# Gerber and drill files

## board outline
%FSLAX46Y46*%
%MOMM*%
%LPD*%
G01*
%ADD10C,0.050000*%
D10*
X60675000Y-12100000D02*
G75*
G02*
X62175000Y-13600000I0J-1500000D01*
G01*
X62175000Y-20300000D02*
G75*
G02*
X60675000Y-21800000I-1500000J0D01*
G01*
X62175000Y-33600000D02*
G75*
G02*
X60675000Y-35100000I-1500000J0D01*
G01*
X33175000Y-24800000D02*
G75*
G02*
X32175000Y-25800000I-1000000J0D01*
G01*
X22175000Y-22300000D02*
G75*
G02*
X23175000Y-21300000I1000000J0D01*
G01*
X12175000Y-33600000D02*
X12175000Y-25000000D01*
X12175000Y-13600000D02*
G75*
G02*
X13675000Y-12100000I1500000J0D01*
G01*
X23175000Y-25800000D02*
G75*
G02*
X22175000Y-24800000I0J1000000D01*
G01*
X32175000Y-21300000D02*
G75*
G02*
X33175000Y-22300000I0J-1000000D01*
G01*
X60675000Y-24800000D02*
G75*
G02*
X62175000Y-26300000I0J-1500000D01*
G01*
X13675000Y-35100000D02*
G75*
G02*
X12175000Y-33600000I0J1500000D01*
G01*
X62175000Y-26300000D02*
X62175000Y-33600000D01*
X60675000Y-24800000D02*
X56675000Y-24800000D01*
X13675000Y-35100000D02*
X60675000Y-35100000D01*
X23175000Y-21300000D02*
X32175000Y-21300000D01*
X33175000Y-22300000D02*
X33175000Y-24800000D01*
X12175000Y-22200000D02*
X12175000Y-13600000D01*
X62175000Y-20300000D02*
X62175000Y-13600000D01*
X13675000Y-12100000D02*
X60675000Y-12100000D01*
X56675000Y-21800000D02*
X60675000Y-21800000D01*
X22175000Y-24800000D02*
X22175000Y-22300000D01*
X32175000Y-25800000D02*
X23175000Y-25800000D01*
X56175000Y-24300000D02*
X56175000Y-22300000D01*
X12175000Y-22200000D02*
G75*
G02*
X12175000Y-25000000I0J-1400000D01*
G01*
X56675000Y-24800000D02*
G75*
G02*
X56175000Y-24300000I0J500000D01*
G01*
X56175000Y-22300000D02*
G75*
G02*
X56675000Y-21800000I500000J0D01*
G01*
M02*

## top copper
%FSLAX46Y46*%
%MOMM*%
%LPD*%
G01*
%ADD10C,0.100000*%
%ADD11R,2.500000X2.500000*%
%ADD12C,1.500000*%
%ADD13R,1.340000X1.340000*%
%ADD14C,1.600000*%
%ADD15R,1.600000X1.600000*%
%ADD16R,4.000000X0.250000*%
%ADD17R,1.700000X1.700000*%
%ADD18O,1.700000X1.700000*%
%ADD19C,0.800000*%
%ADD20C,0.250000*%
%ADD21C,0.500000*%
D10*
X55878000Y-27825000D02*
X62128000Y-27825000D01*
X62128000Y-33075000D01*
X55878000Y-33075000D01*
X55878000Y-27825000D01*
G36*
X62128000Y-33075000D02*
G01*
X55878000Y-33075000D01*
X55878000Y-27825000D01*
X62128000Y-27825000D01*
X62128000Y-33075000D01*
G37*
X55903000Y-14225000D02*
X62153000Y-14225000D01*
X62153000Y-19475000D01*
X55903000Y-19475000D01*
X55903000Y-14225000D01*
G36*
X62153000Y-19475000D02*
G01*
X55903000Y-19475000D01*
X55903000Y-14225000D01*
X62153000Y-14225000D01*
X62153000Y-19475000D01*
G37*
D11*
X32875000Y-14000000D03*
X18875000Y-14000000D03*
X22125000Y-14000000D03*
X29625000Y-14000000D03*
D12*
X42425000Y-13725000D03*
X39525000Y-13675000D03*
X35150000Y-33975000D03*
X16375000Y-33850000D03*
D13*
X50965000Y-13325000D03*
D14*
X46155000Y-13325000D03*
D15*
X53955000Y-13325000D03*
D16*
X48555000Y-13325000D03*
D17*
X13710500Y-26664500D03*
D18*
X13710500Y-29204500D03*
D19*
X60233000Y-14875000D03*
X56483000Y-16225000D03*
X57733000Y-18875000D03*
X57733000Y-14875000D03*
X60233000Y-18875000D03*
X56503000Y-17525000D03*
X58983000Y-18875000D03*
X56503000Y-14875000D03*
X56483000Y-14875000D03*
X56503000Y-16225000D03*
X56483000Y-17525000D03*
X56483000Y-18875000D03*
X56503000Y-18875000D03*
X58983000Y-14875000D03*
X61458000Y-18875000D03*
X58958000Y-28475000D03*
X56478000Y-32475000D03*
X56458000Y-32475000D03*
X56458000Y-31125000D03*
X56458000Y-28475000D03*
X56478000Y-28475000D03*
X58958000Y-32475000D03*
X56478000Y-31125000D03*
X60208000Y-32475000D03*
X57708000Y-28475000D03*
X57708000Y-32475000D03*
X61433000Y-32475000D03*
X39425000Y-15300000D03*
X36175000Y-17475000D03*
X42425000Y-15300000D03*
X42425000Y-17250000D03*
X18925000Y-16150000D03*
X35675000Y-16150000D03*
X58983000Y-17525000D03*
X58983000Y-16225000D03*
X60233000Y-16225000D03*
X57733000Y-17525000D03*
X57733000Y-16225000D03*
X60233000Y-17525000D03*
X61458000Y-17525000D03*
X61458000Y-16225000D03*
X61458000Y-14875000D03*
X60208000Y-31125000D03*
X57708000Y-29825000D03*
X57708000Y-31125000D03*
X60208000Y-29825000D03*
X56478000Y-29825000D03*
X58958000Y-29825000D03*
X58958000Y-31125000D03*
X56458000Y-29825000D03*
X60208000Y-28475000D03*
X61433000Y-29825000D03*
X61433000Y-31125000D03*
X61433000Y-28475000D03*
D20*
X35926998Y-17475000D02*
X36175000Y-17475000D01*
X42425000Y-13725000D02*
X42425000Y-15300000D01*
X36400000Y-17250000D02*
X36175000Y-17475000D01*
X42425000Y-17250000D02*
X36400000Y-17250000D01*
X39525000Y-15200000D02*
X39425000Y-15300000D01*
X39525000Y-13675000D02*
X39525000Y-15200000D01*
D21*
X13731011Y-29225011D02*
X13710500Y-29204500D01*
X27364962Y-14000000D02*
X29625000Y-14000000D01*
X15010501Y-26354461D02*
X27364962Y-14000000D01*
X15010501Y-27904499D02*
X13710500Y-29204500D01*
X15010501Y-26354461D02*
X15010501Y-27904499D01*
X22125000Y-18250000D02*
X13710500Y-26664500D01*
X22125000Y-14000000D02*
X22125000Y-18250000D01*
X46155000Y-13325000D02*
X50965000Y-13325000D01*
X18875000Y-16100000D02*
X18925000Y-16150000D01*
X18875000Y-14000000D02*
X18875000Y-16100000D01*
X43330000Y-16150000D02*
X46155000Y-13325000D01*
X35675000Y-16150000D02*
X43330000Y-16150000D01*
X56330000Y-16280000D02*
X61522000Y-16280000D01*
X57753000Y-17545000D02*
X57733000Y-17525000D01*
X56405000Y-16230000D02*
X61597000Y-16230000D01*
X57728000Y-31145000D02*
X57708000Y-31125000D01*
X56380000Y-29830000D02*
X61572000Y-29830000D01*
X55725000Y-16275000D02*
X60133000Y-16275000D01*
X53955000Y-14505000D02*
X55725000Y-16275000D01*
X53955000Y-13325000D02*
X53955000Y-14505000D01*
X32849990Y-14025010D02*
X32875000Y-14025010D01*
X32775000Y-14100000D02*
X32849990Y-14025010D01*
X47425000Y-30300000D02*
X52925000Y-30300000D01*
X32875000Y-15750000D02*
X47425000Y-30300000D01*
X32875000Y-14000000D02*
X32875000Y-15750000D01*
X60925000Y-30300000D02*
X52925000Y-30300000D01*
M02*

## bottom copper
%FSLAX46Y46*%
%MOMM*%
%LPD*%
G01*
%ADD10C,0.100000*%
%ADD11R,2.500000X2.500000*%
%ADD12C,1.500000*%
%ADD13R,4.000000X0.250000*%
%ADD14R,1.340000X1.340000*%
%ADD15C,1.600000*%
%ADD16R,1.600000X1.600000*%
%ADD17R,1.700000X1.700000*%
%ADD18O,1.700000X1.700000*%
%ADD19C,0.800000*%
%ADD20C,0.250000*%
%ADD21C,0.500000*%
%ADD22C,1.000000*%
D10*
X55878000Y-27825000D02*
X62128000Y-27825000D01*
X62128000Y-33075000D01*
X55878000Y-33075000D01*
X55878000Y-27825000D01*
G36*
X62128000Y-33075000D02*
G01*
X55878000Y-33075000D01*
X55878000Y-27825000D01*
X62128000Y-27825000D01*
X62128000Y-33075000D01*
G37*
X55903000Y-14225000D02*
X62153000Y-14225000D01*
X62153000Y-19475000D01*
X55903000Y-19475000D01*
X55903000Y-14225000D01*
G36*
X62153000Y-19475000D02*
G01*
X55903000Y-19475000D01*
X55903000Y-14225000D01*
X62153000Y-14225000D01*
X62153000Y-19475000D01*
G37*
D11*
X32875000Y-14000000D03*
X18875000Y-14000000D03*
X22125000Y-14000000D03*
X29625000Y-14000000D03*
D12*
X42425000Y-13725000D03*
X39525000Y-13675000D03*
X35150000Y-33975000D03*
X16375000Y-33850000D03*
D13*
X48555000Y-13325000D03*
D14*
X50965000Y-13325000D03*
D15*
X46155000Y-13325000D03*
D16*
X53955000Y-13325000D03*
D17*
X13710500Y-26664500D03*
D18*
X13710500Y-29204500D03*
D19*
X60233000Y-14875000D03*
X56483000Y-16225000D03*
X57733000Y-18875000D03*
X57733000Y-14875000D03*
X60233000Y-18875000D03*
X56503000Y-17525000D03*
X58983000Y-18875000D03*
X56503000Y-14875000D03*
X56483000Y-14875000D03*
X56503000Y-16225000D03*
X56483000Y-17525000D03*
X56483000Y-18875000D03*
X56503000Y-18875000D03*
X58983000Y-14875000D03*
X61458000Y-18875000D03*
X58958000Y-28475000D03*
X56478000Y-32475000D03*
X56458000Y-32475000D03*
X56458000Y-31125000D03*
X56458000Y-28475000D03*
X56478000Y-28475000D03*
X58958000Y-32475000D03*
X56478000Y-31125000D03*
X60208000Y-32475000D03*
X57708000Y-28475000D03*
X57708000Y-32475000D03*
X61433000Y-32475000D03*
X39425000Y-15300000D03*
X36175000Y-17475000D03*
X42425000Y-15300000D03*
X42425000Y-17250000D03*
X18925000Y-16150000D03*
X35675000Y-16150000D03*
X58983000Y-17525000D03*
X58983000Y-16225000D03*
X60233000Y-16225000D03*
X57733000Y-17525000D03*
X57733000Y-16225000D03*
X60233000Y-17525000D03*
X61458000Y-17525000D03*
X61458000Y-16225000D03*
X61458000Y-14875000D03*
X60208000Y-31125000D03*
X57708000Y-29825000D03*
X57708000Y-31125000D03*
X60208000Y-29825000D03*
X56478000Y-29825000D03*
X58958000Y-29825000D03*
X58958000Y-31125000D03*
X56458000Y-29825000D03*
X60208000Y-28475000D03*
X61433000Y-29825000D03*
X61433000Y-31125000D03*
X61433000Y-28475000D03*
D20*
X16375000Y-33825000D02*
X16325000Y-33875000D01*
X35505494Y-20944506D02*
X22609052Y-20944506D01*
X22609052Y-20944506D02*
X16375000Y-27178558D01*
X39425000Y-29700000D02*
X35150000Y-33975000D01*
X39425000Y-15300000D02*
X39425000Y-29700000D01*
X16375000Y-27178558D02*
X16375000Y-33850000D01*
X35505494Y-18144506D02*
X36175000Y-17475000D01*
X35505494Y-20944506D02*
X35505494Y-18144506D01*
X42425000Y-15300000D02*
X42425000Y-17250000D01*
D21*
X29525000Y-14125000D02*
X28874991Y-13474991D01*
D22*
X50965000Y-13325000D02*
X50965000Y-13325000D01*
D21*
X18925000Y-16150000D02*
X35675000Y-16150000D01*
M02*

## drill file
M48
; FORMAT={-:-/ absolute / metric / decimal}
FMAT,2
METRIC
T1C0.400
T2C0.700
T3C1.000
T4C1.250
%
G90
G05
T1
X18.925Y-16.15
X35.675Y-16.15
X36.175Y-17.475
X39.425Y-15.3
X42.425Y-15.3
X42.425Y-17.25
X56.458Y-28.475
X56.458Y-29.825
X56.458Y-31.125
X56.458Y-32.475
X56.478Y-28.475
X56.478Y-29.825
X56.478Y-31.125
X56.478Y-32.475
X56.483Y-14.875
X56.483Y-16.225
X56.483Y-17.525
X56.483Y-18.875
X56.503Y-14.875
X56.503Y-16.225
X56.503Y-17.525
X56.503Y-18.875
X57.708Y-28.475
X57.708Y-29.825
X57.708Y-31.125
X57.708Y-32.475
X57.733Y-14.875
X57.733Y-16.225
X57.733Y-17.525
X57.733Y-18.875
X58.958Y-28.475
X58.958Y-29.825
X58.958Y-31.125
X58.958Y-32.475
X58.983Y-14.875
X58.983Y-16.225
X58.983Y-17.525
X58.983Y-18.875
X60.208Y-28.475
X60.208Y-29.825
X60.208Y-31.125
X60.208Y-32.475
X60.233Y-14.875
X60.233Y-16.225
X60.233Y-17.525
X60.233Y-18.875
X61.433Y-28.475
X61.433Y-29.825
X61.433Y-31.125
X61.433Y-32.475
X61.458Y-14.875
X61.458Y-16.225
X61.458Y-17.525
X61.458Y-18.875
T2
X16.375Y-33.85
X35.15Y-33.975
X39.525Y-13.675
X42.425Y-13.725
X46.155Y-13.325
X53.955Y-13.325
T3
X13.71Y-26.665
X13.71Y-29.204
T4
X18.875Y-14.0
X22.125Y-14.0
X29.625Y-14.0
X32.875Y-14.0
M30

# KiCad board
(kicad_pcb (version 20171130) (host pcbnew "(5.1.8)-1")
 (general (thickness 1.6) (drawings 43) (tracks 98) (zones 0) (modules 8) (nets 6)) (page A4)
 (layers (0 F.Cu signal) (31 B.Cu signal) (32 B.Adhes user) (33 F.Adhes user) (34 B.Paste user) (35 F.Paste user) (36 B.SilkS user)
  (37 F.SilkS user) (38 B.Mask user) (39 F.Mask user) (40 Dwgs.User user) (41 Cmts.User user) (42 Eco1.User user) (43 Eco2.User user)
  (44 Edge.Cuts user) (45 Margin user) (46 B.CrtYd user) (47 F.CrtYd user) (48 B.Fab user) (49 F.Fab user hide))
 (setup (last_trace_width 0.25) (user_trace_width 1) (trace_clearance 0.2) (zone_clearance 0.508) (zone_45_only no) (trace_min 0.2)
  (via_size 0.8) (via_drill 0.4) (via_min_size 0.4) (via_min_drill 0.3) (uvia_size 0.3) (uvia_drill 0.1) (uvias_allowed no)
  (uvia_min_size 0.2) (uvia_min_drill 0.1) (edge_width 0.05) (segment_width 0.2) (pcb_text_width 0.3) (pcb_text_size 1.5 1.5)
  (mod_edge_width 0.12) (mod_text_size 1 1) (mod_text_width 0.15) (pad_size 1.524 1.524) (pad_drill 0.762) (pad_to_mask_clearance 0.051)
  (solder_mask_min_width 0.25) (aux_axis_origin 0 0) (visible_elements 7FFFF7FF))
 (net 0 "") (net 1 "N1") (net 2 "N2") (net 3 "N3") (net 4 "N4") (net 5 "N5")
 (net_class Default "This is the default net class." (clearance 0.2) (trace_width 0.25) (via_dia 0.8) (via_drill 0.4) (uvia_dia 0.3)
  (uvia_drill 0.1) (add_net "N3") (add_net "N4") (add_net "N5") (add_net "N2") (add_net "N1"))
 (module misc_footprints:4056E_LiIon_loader (layer F.Cu) (at 25.875 25 90)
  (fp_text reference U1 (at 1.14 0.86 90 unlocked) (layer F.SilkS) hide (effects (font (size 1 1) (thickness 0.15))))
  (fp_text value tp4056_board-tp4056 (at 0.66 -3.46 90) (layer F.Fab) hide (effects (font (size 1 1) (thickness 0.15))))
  (pad 6 thru_hole rect (at 11 7 90) (size 2.5 2.5) (drill 1.25) (layers *.Cu *.Mask F.SilkS) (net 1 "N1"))
  (pad 5 thru_hole rect (at 11 -7 90) (size 2.5 2.5) (drill 1.25) (layers *.Cu *.Mask F.SilkS) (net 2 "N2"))
  (pad 3 thru_hole rect (at 11 -3.75 90) (size 2.5 2.5) (drill 1.25) (layers *.Cu *.Mask F.SilkS) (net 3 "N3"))
  (pad 4 thru_hole rect (at 11 3.75 90) (size 2.5 2.5) (drill 1.25) (layers *.Cu *.Mask F.SilkS) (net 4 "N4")))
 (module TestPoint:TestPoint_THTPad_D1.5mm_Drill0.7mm (layer F.Cu) (at 42.425 13.725)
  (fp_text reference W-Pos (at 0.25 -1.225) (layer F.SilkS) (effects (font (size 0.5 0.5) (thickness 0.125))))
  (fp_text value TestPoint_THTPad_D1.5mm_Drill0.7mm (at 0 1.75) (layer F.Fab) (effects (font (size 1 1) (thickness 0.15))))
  (pad 1 thru_hole circle (at 0 0) (size 1.5 1.5) (drill 0.7) (layers *.Cu *.Mask)))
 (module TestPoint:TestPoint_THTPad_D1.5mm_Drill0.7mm (layer F.Cu) (at 39.525 13.675)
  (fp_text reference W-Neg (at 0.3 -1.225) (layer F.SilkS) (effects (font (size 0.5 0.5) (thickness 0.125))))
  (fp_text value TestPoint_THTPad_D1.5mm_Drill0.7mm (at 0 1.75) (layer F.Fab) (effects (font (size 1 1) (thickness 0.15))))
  (pad 1 thru_hole circle (at 0 0) (size 1.5 1.5) (drill 0.7) (layers *.Cu *.Mask)))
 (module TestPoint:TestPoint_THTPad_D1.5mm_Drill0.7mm (layer F.Cu) (at 35.15 33.975)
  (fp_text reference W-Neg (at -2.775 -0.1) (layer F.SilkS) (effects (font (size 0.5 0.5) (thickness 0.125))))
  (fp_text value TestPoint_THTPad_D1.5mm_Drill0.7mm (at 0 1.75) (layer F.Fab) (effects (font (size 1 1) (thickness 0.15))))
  (pad 1 thru_hole circle (at 0 0) (size 1.5 1.5) (drill 0.7) (layers *.Cu *.Mask)))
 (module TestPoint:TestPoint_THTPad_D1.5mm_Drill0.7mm (layer F.Cu) (at 16.375 33.85)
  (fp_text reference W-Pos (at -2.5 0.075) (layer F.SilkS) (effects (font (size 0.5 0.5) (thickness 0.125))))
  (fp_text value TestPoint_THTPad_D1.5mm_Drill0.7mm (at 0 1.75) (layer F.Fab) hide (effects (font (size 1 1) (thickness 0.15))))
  (pad 1 thru_hole circle (at 0 0) (size 1.5 1.5) (drill 0.7) (layers *.Cu *.Mask)))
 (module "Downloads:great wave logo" (layer F.Cu) (at 40.675 30.55)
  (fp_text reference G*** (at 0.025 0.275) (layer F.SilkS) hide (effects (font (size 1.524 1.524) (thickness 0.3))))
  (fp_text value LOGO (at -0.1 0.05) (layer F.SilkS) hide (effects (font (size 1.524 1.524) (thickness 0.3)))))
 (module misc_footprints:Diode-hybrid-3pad (layer F.Cu) (at 50.055 13.325)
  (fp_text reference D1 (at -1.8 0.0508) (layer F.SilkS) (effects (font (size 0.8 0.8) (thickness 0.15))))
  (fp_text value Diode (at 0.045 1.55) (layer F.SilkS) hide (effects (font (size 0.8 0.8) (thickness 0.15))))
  (pad 2 smd rect (at -1.5 0) (size 4 0.25) (layers B.Cu) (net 2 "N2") (solder_mask_margin -999))
  (pad 2 smd rect (at 0.91 0) (size 1.34 1.34) (layers B.Cu B.Paste B.Mask) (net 2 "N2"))
  (pad 2 smd rect (at 0.91 0) (size 1.34 1.34) (layers F.Cu F.Paste F.Mask) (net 2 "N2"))
  (pad 2 thru_hole circle (at -3.9 0) (size 1.6 1.6) (drill 0.7) (layers *.Cu *.Mask F.SilkS) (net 2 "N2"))
  (pad 1 thru_hole rect (at 3.9 0) (size 1.6 1.6) (drill 0.7) (layers *.Cu *.Mask F.SilkS) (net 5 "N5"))
  (pad 2 smd rect (at -1.5 0) (size 4 0.25) (layers F.Cu) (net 2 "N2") (solder_mask_margin -999)))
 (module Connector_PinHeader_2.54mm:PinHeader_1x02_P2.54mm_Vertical (layer F.Cu) (at 13.7105 26.6645)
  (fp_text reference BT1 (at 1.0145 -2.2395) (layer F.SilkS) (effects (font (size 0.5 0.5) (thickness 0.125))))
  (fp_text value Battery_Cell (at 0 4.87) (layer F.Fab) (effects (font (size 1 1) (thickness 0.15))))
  (pad 1 thru_hole rect (at 0 0) (size 1.7 1.7) (drill 1) (layers *.Cu *.Mask) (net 3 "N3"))
  (pad 2 thru_hole oval (at 0 2.54) (size 1.7 1.7) (drill 1) (layers *.Cu *.Mask) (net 4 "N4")))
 (gr_arc (start 60.675 13.6) (end 62.175 13.6) (angle -90) (layer Edge.Cuts) (width 0.05))
 (gr_arc (start 60.675 20.3) (end 60.675 21.8) (angle -90) (layer Edge.Cuts) (width 0.05))
 (gr_arc (start 60.675 33.6) (end 60.675 35.1) (angle -90) (layer Edge.Cuts) (width 0.05))
 (gr_arc (start 32.175 24.8) (end 32.175 25.8) (angle -90) (layer Edge.Cuts) (width 0.05))
 (gr_arc (start 23.175 22.3) (end 23.175 21.3) (angle -90) (layer Edge.Cuts) (width 0.05))
 (gr_line (start 12.175 33.6) (end 12.175 25) (layer Edge.Cuts) (width 0.05))
 (gr_arc (start 13.675 13.6) (end 13.675 12.1) (angle -90) (layer Edge.Cuts) (width 0.05))
 (gr_arc (start 23.175 24.8) (end 22.175 24.8) (angle -90) (layer Edge.Cuts) (width 0.05))
 (gr_arc (start 32.175 22.3) (end 33.175 22.3) (angle -90) (layer Edge.Cuts) (width 0.05))
 (gr_arc (start 60.675 26.3) (end 62.175 26.3) (angle -90) (layer Edge.Cuts) (width 0.05))
 (gr_arc (start 13.675 33.6) (end 12.175 33.6) (angle -90) (layer Edge.Cuts) (width 0.05))
 (gr_line (start 62.175 26.3) (end 62.175 33.6) (layer Edge.Cuts) (width 0.05))
 (gr_line (start 60.675 24.8) (end 56.675 24.8) (layer Edge.Cuts) (width 0.05))
 (gr_line (start 13.675 35.1) (end 60.675 35.1) (layer Edge.Cuts) (width 0.05))
 (gr_line (start 23.175 21.3) (end 32.175 21.3) (layer Edge.Cuts) (width 0.05))
 (gr_line (start 33.175 22.3) (end 33.175 24.8) (layer Edge.Cuts) (width 0.05))
 (gr_line (start 12.175 22.2) (end 12.175 13.6) (layer Edge.Cuts) (width 0.05))
 (gr_line (start 62.175 20.3) (end 62.175 13.6) (layer Edge.Cuts) (width 0.05))
 (gr_line (start 13.675 12.1) (end 60.675 12.1) (layer Edge.Cuts) (width 0.05))
 (gr_line (start 56.675 21.8) (end 60.675 21.8) (layer Edge.Cuts) (width 0.05))
 (gr_line (start 22.175 24.8) (end 22.175 22.3) (layer Edge.Cuts) (width 0.05))
 (gr_line (start 32.175 25.8) (end 23.175 25.8) (layer Edge.Cuts) (width 0.05))
 (gr_line (start 56.175 24.3) (end 56.175 22.3) (layer Edge.Cuts) (width 0.05))
 (gr_arc (start 12.175 23.6) (end 12.175 25) (angle -180) (layer Edge.Cuts) (width 0.05))
 (gr_arc (start 56.675 24.3) (end 56.175 24.3) (angle -90) (layer Edge.Cuts) (width 0.05))
 (gr_arc (start 56.675 22.3) (end 56.675 21.8) (angle -90) (layer Edge.Cuts) (width 0.05))
 (gr_poly (pts (xy 55.878 27.825) (xy 62.128 27.825) (xy 62.128 33.075) (xy 55.878 33.075)) (layer F.Cu) (width 0.1))
 (gr_poly (pts (xy 55.878 27.825) (xy 62.128 27.825) (xy 62.128 33.075) (xy 55.878 33.075)) (layer B.Cu) (width 0.1))
 (gr_poly (pts (xy 55.903 14.225) (xy 62.153 14.225) (xy 62.153 19.475) (xy 55.903 19.475)) (layer F.Cu) (width 0.1))
 (gr_poly (pts (xy 55.903 14.225) (xy 62.153 14.225) (xy 62.153 19.475) (xy 55.903 19.475)) (layer B.Cu) (width 0.1))
 (via (at 60.233 14.875) (size 0.8) (drill 0.4) (layers F.Cu B.Cu) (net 5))
 (via (at 56.483 16.225) (size 0.8) (drill 0.4) (layers F.Cu B.Cu) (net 5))
 (via (at 57.733 18.875) (size 0.8) (drill 0.4) (layers F.Cu B.Cu) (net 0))
 (via (at 57.733 14.875) (size 0.8) (drill 0.4) (layers F.Cu B.Cu) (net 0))
 (via (at 60.233 18.875) (size 0.8) (drill 0.4) (layers F.Cu B.Cu) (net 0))
 (via (at 56.503 17.525) (size 0.8) (drill 0.4) (layers F.Cu B.Cu) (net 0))
 (via (at 58.983 18.875) (size 0.8) (drill 0.4) (layers F.Cu B.Cu) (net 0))
 (via (at 56.503 14.875) (size 0.8) (drill 0.4) (layers F.Cu B.Cu) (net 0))
 (via (at 56.483 14.875) (size 0.8) (drill 0.4) (layers F.Cu B.Cu) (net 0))
 (via (at 56.503 16.225) (size 0.8) (drill 0.4) (layers F.Cu B.Cu) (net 5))
 (via (at 56.483 17.525) (size 0.8) (drill 0.4) (layers F.Cu B.Cu) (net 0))
 (via (at 56.483 18.875) (size 0.8) (drill 0.4) (layers F.Cu B.Cu) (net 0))
 (via (at 56.503 18.875) (size 0.8) (drill 0.4) (layers F.Cu B.Cu) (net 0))
 (via (at 58.983 14.875) (size 0.8) (drill 0.4) (layers F.Cu B.Cu) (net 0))
 (via (at 61.458 18.875) (size 0.8) (drill 0.4) (layers F.Cu B.Cu) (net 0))
 (via (at 58.958 28.475) (size 0.8) (drill 0.4) (layers F.Cu B.Cu) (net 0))
 (via (at 56.478 32.475) (size 0.8) (drill 0.4) (layers F.Cu B.Cu) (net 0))
 (via (at 56.458 32.475) (size 0.8) (drill 0.4) (layers F.Cu B.Cu) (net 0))
 (via (at 56.458 31.125) (size 0.8) (drill 0.4) (layers F.Cu B.Cu) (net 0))
 (via (at 56.458 28.475) (size 0.8) (drill 0.4) (layers F.Cu B.Cu) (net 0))
 (via (at 56.478 28.475) (size 0.8) (drill 0.4) (layers F.Cu B.Cu) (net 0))
 (via (at 58.958 32.475) (size 0.8) (drill 0.4) (layers F.Cu B.Cu) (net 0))
 (via (at 56.478 31.125) (size 0.8) (drill 0.4) (layers F.Cu B.Cu) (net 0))
 (via (at 60.208 32.475) (size 0.8) (drill 0.4) (layers F.Cu B.Cu) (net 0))
 (via (at 57.708 28.475) (size 0.8) (drill 0.4) (layers F.Cu B.Cu) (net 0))
 (via (at 57.708 32.475) (size 0.8) (drill 0.4) (layers F.Cu B.Cu) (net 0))
 (via (at 61.433 32.475) (size 0.8) (drill 0.4) (layers F.Cu B.Cu) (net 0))
 (via (at 39.425 15.3) (size 0.8) (drill 0.4) (layers F.Cu B.Cu) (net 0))
 (segment (start 16.375 33.825) (end 16.325 33.875) (width 0.25) (layer B.Cu) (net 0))
 (segment (start 35.926998 17.475) (end 36.175 17.475) (width 0.25) (layer F.Cu) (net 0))
 (via (at 36.175 17.475) (size 0.8) (drill 0.4) (layers F.Cu B.Cu) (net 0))
 (segment (start 35.505494 20.944506) (end 22.609052 20.944506) (width 0.25) (layer B.Cu) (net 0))
 (segment (start 22.609052 20.944506) (end 16.375 27.178558) (width 0.25) (layer B.Cu) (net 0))
 (segment (start 39.425 29.7) (end 35.15 33.975) (width 0.25) (layer B.Cu) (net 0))
 (segment (start 39.425 15.3) (end 39.425 29.7) (width 0.25) (layer B.Cu) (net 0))
 (segment (start 16.375 27.178558) (end 16.375 33.85) (width 0.25) (layer B.Cu) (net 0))
 (segment (start 35.505494 18.144506) (end 36.175 17.475) (width 0.25) (layer B.Cu) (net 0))
 (segment (start 35.505494 20.944506) (end 35.505494 18.144506) (width 0.25) (layer B.Cu) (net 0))
 (via (at 42.425 15.3) (size 0.8) (drill 0.4) (layers F.Cu B.Cu) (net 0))
 (segment (start 42.425 13.725) (end 42.425 15.3) (width 0.25) (layer F.Cu) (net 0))
 (via (at 42.425 17.25) (size 0.8) (drill 0.4) (layers F.Cu B.Cu) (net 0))
 (segment (start 42.425 15.3) (end 42.425 17.25) (width 0.25) (layer B.Cu) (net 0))
 (segment (start 36.4 17.25) (end 36.175 17.475) (width 0.25) (layer F.Cu) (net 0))
 (segment (start 42.425 17.25) (end 36.4 17.25) (width 0.25) (layer F.Cu) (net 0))
 (segment (start 39.525 15.2) (end 39.425 15.3) (width 0.25) (layer F.Cu) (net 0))
 (segment (start 39.525 13.675) (end 39.525 15.2) (width 0.25) (layer F.Cu) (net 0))
 (segment (start 29.525 14.125) (end 28.874991 13.474991) (width 0.5) (layer B.Cu) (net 4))
 (segment (start 13.731011 29.225011) (end 13.7105 29.2045) (width 0.5) (layer F.Cu) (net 4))
 (segment (start 27.364962 14) (end 29.625 14) (width 0.5) (layer F.Cu) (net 4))
 (segment (start 15.010501 26.354461) (end 27.364962 14) (width 0.5) (layer F.Cu) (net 4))
 (segment (start 15.010501 27.904499) (end 13.7105 29.2045) (width 0.5) (layer F.Cu) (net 4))
 (segment (start 15.010501 26.354461) (end 15.010501 27.904499) (width 0.5) (layer F.Cu) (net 4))
 (segment (start 22.125 18.25) (end 13.7105 26.6645) (width 0.5) (layer F.Cu) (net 3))
 (segment (start 22.125 14) (end 22.125 18.25) (width 0.5) (layer F.Cu) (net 3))
 (segment (start 50.965 13.325) (end 50.965 13.325) (width 1) (layer B.Cu) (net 2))
 (segment (start 46.155 13.325) (end 50.965 13.325) (width 0.5) (layer F.Cu) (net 2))
 (via (at 18.925 16.15) (size 0.8) (drill 0.4) (layers F.Cu B.Cu) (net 2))
 (segment (start 18.875 16.1) (end 18.925 16.15) (width 0.5) (layer F.Cu) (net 2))
 (segment (start 18.875 14) (end 18.875 16.1) (width 0.5) (layer F.Cu) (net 2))
 (segment (start 18.925 16.15) (end 35.675 16.15) (width 0.5) (layer B.Cu) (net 2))
 (via (at 35.675 16.15) (size 0.8) (drill 0.4) (layers F.Cu B.Cu) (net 2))
 (segment (start 43.33 16.15) (end 46.155 13.325) (width 0.5) (layer F.Cu) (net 2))
 (segment (start 35.675 16.15) (end 43.33 16.15) (width 0.5) (layer F.Cu) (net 2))
 (segment (start 56.33 16.28) (end 61.522 16.28) (width 0.5) (layer F.Cu) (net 5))
 (via (at 58.983 17.525) (size 0.8) (drill 0.4) (layers F.Cu B.Cu) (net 5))
 (segment (start 57.753 17.545) (end 57.733 17.525) (width 0.5) (layer F.Cu) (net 5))
 (via (at 58.983 16.225) (size 0.8) (drill 0.4) (layers F.Cu B.Cu) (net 5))
 (via (at 60.233 16.225) (size 0.8) (drill 0.4) (layers F.Cu B.Cu) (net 5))
 (via (at 57.733 17.525) (size 0.8) (drill 0.4) (layers F.Cu B.Cu) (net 5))
 (via (at 57.733 16.225) (size 0.8) (drill 0.4) (layers F.Cu B.Cu) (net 5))
 (via (at 60.233 17.525) (size 0.8) (drill 0.4) (layers F.Cu B.Cu) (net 5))
 (via (at 61.458 17.525) (size 0.8) (drill 0.4) (layers F.Cu B.Cu) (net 5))
 (via (at 61.458 16.225) (size 0.8) (drill 0.4) (layers F.Cu B.Cu) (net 5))
 (segment (start 56.405 16.23) (end 61.597 16.23) (width 0.5) (layer F.Cu) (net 5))
 (via (at 61.458 14.875) (size 0.8) (drill 0.4) (layers F.Cu B.Cu) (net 5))
 (via (at 60.208 31.125) (size 0.8) (drill 0.4) (layers F.Cu B.Cu) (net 5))
 (via (at 57.708 29.825) (size 0.8) (drill 0.4) (layers F.Cu B.Cu) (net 5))
 (via (at 57.708 31.125) (size 0.8) (drill 0.4) (layers F.Cu B.Cu) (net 5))
 (via (at 60.208 29.825) (size 0.8) (drill 0.4) (layers F.Cu B.Cu) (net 5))
 (via (at 56.478 29.825) (size 0.8) (drill 0.4) (layers F.Cu B.Cu) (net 5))
 (via (at 58.958 29.825) (size 0.8) (drill 0.4) (layers F.Cu B.Cu) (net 5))
 (segment (start 57.728 31.145) (end 57.708 31.125) (width 0.5) (layer F.Cu) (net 5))
 (via (at 58.958 31.125) (size 0.8) (drill 0.4) (layers F.Cu B.Cu) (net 5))
 (segment (start 56.38 29.83) (end 61.572 29.83) (width 0.5) (layer F.Cu) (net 5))
 (via (at 56.458 29.825) (size 0.8) (drill 0.4) (layers F.Cu B.Cu) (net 5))
 (via (at 60.208 28.475) (size 0.8) (drill 0.4) (layers F.Cu B.Cu) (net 5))
 (via (at 61.433 29.825) (size 0.8) (drill 0.4) (layers F.Cu B.Cu) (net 5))
 (via (at 61.433 31.125) (size 0.8) (drill 0.4) (layers F.Cu B.Cu) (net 5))
 (via (at 61.433 28.475) (size 0.8) (drill 0.4) (layers F.Cu B.Cu) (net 5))
 (segment (start 55.725 16.275) (end 60.133 16.275) (width 0.5) (layer F.Cu) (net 5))
 (segment (start 53.955 14.505) (end 55.725 16.275) (width 0.5) (layer F.Cu) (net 5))
 (segment (start 53.955 13.325) (end 53.955 14.505) (width 0.5) (layer F.Cu) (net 5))
 (segment (start 32.84999 14.02501) (end 32.875 14.02501) (width 0.5) (layer F.Cu) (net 1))
 (segment (start 32.775 14.1) (end 32.84999 14.02501) (width 0.5) (layer F.Cu) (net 1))
 (segment (start 47.425 30.3) (end 52.925 30.3) (width 0.5) (layer F.Cu) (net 1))
 (segment (start 32.875 15.75) (end 47.425 30.3) (width 0.5) (layer F.Cu) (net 1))
 (segment (start 32.875 14) (end 32.875 15.75) (width 0.5) (layer F.Cu) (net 1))
 (segment (start 60.925 30.3) (end 52.925 30.3) (width 0.5) (layer F.Cu) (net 1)))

